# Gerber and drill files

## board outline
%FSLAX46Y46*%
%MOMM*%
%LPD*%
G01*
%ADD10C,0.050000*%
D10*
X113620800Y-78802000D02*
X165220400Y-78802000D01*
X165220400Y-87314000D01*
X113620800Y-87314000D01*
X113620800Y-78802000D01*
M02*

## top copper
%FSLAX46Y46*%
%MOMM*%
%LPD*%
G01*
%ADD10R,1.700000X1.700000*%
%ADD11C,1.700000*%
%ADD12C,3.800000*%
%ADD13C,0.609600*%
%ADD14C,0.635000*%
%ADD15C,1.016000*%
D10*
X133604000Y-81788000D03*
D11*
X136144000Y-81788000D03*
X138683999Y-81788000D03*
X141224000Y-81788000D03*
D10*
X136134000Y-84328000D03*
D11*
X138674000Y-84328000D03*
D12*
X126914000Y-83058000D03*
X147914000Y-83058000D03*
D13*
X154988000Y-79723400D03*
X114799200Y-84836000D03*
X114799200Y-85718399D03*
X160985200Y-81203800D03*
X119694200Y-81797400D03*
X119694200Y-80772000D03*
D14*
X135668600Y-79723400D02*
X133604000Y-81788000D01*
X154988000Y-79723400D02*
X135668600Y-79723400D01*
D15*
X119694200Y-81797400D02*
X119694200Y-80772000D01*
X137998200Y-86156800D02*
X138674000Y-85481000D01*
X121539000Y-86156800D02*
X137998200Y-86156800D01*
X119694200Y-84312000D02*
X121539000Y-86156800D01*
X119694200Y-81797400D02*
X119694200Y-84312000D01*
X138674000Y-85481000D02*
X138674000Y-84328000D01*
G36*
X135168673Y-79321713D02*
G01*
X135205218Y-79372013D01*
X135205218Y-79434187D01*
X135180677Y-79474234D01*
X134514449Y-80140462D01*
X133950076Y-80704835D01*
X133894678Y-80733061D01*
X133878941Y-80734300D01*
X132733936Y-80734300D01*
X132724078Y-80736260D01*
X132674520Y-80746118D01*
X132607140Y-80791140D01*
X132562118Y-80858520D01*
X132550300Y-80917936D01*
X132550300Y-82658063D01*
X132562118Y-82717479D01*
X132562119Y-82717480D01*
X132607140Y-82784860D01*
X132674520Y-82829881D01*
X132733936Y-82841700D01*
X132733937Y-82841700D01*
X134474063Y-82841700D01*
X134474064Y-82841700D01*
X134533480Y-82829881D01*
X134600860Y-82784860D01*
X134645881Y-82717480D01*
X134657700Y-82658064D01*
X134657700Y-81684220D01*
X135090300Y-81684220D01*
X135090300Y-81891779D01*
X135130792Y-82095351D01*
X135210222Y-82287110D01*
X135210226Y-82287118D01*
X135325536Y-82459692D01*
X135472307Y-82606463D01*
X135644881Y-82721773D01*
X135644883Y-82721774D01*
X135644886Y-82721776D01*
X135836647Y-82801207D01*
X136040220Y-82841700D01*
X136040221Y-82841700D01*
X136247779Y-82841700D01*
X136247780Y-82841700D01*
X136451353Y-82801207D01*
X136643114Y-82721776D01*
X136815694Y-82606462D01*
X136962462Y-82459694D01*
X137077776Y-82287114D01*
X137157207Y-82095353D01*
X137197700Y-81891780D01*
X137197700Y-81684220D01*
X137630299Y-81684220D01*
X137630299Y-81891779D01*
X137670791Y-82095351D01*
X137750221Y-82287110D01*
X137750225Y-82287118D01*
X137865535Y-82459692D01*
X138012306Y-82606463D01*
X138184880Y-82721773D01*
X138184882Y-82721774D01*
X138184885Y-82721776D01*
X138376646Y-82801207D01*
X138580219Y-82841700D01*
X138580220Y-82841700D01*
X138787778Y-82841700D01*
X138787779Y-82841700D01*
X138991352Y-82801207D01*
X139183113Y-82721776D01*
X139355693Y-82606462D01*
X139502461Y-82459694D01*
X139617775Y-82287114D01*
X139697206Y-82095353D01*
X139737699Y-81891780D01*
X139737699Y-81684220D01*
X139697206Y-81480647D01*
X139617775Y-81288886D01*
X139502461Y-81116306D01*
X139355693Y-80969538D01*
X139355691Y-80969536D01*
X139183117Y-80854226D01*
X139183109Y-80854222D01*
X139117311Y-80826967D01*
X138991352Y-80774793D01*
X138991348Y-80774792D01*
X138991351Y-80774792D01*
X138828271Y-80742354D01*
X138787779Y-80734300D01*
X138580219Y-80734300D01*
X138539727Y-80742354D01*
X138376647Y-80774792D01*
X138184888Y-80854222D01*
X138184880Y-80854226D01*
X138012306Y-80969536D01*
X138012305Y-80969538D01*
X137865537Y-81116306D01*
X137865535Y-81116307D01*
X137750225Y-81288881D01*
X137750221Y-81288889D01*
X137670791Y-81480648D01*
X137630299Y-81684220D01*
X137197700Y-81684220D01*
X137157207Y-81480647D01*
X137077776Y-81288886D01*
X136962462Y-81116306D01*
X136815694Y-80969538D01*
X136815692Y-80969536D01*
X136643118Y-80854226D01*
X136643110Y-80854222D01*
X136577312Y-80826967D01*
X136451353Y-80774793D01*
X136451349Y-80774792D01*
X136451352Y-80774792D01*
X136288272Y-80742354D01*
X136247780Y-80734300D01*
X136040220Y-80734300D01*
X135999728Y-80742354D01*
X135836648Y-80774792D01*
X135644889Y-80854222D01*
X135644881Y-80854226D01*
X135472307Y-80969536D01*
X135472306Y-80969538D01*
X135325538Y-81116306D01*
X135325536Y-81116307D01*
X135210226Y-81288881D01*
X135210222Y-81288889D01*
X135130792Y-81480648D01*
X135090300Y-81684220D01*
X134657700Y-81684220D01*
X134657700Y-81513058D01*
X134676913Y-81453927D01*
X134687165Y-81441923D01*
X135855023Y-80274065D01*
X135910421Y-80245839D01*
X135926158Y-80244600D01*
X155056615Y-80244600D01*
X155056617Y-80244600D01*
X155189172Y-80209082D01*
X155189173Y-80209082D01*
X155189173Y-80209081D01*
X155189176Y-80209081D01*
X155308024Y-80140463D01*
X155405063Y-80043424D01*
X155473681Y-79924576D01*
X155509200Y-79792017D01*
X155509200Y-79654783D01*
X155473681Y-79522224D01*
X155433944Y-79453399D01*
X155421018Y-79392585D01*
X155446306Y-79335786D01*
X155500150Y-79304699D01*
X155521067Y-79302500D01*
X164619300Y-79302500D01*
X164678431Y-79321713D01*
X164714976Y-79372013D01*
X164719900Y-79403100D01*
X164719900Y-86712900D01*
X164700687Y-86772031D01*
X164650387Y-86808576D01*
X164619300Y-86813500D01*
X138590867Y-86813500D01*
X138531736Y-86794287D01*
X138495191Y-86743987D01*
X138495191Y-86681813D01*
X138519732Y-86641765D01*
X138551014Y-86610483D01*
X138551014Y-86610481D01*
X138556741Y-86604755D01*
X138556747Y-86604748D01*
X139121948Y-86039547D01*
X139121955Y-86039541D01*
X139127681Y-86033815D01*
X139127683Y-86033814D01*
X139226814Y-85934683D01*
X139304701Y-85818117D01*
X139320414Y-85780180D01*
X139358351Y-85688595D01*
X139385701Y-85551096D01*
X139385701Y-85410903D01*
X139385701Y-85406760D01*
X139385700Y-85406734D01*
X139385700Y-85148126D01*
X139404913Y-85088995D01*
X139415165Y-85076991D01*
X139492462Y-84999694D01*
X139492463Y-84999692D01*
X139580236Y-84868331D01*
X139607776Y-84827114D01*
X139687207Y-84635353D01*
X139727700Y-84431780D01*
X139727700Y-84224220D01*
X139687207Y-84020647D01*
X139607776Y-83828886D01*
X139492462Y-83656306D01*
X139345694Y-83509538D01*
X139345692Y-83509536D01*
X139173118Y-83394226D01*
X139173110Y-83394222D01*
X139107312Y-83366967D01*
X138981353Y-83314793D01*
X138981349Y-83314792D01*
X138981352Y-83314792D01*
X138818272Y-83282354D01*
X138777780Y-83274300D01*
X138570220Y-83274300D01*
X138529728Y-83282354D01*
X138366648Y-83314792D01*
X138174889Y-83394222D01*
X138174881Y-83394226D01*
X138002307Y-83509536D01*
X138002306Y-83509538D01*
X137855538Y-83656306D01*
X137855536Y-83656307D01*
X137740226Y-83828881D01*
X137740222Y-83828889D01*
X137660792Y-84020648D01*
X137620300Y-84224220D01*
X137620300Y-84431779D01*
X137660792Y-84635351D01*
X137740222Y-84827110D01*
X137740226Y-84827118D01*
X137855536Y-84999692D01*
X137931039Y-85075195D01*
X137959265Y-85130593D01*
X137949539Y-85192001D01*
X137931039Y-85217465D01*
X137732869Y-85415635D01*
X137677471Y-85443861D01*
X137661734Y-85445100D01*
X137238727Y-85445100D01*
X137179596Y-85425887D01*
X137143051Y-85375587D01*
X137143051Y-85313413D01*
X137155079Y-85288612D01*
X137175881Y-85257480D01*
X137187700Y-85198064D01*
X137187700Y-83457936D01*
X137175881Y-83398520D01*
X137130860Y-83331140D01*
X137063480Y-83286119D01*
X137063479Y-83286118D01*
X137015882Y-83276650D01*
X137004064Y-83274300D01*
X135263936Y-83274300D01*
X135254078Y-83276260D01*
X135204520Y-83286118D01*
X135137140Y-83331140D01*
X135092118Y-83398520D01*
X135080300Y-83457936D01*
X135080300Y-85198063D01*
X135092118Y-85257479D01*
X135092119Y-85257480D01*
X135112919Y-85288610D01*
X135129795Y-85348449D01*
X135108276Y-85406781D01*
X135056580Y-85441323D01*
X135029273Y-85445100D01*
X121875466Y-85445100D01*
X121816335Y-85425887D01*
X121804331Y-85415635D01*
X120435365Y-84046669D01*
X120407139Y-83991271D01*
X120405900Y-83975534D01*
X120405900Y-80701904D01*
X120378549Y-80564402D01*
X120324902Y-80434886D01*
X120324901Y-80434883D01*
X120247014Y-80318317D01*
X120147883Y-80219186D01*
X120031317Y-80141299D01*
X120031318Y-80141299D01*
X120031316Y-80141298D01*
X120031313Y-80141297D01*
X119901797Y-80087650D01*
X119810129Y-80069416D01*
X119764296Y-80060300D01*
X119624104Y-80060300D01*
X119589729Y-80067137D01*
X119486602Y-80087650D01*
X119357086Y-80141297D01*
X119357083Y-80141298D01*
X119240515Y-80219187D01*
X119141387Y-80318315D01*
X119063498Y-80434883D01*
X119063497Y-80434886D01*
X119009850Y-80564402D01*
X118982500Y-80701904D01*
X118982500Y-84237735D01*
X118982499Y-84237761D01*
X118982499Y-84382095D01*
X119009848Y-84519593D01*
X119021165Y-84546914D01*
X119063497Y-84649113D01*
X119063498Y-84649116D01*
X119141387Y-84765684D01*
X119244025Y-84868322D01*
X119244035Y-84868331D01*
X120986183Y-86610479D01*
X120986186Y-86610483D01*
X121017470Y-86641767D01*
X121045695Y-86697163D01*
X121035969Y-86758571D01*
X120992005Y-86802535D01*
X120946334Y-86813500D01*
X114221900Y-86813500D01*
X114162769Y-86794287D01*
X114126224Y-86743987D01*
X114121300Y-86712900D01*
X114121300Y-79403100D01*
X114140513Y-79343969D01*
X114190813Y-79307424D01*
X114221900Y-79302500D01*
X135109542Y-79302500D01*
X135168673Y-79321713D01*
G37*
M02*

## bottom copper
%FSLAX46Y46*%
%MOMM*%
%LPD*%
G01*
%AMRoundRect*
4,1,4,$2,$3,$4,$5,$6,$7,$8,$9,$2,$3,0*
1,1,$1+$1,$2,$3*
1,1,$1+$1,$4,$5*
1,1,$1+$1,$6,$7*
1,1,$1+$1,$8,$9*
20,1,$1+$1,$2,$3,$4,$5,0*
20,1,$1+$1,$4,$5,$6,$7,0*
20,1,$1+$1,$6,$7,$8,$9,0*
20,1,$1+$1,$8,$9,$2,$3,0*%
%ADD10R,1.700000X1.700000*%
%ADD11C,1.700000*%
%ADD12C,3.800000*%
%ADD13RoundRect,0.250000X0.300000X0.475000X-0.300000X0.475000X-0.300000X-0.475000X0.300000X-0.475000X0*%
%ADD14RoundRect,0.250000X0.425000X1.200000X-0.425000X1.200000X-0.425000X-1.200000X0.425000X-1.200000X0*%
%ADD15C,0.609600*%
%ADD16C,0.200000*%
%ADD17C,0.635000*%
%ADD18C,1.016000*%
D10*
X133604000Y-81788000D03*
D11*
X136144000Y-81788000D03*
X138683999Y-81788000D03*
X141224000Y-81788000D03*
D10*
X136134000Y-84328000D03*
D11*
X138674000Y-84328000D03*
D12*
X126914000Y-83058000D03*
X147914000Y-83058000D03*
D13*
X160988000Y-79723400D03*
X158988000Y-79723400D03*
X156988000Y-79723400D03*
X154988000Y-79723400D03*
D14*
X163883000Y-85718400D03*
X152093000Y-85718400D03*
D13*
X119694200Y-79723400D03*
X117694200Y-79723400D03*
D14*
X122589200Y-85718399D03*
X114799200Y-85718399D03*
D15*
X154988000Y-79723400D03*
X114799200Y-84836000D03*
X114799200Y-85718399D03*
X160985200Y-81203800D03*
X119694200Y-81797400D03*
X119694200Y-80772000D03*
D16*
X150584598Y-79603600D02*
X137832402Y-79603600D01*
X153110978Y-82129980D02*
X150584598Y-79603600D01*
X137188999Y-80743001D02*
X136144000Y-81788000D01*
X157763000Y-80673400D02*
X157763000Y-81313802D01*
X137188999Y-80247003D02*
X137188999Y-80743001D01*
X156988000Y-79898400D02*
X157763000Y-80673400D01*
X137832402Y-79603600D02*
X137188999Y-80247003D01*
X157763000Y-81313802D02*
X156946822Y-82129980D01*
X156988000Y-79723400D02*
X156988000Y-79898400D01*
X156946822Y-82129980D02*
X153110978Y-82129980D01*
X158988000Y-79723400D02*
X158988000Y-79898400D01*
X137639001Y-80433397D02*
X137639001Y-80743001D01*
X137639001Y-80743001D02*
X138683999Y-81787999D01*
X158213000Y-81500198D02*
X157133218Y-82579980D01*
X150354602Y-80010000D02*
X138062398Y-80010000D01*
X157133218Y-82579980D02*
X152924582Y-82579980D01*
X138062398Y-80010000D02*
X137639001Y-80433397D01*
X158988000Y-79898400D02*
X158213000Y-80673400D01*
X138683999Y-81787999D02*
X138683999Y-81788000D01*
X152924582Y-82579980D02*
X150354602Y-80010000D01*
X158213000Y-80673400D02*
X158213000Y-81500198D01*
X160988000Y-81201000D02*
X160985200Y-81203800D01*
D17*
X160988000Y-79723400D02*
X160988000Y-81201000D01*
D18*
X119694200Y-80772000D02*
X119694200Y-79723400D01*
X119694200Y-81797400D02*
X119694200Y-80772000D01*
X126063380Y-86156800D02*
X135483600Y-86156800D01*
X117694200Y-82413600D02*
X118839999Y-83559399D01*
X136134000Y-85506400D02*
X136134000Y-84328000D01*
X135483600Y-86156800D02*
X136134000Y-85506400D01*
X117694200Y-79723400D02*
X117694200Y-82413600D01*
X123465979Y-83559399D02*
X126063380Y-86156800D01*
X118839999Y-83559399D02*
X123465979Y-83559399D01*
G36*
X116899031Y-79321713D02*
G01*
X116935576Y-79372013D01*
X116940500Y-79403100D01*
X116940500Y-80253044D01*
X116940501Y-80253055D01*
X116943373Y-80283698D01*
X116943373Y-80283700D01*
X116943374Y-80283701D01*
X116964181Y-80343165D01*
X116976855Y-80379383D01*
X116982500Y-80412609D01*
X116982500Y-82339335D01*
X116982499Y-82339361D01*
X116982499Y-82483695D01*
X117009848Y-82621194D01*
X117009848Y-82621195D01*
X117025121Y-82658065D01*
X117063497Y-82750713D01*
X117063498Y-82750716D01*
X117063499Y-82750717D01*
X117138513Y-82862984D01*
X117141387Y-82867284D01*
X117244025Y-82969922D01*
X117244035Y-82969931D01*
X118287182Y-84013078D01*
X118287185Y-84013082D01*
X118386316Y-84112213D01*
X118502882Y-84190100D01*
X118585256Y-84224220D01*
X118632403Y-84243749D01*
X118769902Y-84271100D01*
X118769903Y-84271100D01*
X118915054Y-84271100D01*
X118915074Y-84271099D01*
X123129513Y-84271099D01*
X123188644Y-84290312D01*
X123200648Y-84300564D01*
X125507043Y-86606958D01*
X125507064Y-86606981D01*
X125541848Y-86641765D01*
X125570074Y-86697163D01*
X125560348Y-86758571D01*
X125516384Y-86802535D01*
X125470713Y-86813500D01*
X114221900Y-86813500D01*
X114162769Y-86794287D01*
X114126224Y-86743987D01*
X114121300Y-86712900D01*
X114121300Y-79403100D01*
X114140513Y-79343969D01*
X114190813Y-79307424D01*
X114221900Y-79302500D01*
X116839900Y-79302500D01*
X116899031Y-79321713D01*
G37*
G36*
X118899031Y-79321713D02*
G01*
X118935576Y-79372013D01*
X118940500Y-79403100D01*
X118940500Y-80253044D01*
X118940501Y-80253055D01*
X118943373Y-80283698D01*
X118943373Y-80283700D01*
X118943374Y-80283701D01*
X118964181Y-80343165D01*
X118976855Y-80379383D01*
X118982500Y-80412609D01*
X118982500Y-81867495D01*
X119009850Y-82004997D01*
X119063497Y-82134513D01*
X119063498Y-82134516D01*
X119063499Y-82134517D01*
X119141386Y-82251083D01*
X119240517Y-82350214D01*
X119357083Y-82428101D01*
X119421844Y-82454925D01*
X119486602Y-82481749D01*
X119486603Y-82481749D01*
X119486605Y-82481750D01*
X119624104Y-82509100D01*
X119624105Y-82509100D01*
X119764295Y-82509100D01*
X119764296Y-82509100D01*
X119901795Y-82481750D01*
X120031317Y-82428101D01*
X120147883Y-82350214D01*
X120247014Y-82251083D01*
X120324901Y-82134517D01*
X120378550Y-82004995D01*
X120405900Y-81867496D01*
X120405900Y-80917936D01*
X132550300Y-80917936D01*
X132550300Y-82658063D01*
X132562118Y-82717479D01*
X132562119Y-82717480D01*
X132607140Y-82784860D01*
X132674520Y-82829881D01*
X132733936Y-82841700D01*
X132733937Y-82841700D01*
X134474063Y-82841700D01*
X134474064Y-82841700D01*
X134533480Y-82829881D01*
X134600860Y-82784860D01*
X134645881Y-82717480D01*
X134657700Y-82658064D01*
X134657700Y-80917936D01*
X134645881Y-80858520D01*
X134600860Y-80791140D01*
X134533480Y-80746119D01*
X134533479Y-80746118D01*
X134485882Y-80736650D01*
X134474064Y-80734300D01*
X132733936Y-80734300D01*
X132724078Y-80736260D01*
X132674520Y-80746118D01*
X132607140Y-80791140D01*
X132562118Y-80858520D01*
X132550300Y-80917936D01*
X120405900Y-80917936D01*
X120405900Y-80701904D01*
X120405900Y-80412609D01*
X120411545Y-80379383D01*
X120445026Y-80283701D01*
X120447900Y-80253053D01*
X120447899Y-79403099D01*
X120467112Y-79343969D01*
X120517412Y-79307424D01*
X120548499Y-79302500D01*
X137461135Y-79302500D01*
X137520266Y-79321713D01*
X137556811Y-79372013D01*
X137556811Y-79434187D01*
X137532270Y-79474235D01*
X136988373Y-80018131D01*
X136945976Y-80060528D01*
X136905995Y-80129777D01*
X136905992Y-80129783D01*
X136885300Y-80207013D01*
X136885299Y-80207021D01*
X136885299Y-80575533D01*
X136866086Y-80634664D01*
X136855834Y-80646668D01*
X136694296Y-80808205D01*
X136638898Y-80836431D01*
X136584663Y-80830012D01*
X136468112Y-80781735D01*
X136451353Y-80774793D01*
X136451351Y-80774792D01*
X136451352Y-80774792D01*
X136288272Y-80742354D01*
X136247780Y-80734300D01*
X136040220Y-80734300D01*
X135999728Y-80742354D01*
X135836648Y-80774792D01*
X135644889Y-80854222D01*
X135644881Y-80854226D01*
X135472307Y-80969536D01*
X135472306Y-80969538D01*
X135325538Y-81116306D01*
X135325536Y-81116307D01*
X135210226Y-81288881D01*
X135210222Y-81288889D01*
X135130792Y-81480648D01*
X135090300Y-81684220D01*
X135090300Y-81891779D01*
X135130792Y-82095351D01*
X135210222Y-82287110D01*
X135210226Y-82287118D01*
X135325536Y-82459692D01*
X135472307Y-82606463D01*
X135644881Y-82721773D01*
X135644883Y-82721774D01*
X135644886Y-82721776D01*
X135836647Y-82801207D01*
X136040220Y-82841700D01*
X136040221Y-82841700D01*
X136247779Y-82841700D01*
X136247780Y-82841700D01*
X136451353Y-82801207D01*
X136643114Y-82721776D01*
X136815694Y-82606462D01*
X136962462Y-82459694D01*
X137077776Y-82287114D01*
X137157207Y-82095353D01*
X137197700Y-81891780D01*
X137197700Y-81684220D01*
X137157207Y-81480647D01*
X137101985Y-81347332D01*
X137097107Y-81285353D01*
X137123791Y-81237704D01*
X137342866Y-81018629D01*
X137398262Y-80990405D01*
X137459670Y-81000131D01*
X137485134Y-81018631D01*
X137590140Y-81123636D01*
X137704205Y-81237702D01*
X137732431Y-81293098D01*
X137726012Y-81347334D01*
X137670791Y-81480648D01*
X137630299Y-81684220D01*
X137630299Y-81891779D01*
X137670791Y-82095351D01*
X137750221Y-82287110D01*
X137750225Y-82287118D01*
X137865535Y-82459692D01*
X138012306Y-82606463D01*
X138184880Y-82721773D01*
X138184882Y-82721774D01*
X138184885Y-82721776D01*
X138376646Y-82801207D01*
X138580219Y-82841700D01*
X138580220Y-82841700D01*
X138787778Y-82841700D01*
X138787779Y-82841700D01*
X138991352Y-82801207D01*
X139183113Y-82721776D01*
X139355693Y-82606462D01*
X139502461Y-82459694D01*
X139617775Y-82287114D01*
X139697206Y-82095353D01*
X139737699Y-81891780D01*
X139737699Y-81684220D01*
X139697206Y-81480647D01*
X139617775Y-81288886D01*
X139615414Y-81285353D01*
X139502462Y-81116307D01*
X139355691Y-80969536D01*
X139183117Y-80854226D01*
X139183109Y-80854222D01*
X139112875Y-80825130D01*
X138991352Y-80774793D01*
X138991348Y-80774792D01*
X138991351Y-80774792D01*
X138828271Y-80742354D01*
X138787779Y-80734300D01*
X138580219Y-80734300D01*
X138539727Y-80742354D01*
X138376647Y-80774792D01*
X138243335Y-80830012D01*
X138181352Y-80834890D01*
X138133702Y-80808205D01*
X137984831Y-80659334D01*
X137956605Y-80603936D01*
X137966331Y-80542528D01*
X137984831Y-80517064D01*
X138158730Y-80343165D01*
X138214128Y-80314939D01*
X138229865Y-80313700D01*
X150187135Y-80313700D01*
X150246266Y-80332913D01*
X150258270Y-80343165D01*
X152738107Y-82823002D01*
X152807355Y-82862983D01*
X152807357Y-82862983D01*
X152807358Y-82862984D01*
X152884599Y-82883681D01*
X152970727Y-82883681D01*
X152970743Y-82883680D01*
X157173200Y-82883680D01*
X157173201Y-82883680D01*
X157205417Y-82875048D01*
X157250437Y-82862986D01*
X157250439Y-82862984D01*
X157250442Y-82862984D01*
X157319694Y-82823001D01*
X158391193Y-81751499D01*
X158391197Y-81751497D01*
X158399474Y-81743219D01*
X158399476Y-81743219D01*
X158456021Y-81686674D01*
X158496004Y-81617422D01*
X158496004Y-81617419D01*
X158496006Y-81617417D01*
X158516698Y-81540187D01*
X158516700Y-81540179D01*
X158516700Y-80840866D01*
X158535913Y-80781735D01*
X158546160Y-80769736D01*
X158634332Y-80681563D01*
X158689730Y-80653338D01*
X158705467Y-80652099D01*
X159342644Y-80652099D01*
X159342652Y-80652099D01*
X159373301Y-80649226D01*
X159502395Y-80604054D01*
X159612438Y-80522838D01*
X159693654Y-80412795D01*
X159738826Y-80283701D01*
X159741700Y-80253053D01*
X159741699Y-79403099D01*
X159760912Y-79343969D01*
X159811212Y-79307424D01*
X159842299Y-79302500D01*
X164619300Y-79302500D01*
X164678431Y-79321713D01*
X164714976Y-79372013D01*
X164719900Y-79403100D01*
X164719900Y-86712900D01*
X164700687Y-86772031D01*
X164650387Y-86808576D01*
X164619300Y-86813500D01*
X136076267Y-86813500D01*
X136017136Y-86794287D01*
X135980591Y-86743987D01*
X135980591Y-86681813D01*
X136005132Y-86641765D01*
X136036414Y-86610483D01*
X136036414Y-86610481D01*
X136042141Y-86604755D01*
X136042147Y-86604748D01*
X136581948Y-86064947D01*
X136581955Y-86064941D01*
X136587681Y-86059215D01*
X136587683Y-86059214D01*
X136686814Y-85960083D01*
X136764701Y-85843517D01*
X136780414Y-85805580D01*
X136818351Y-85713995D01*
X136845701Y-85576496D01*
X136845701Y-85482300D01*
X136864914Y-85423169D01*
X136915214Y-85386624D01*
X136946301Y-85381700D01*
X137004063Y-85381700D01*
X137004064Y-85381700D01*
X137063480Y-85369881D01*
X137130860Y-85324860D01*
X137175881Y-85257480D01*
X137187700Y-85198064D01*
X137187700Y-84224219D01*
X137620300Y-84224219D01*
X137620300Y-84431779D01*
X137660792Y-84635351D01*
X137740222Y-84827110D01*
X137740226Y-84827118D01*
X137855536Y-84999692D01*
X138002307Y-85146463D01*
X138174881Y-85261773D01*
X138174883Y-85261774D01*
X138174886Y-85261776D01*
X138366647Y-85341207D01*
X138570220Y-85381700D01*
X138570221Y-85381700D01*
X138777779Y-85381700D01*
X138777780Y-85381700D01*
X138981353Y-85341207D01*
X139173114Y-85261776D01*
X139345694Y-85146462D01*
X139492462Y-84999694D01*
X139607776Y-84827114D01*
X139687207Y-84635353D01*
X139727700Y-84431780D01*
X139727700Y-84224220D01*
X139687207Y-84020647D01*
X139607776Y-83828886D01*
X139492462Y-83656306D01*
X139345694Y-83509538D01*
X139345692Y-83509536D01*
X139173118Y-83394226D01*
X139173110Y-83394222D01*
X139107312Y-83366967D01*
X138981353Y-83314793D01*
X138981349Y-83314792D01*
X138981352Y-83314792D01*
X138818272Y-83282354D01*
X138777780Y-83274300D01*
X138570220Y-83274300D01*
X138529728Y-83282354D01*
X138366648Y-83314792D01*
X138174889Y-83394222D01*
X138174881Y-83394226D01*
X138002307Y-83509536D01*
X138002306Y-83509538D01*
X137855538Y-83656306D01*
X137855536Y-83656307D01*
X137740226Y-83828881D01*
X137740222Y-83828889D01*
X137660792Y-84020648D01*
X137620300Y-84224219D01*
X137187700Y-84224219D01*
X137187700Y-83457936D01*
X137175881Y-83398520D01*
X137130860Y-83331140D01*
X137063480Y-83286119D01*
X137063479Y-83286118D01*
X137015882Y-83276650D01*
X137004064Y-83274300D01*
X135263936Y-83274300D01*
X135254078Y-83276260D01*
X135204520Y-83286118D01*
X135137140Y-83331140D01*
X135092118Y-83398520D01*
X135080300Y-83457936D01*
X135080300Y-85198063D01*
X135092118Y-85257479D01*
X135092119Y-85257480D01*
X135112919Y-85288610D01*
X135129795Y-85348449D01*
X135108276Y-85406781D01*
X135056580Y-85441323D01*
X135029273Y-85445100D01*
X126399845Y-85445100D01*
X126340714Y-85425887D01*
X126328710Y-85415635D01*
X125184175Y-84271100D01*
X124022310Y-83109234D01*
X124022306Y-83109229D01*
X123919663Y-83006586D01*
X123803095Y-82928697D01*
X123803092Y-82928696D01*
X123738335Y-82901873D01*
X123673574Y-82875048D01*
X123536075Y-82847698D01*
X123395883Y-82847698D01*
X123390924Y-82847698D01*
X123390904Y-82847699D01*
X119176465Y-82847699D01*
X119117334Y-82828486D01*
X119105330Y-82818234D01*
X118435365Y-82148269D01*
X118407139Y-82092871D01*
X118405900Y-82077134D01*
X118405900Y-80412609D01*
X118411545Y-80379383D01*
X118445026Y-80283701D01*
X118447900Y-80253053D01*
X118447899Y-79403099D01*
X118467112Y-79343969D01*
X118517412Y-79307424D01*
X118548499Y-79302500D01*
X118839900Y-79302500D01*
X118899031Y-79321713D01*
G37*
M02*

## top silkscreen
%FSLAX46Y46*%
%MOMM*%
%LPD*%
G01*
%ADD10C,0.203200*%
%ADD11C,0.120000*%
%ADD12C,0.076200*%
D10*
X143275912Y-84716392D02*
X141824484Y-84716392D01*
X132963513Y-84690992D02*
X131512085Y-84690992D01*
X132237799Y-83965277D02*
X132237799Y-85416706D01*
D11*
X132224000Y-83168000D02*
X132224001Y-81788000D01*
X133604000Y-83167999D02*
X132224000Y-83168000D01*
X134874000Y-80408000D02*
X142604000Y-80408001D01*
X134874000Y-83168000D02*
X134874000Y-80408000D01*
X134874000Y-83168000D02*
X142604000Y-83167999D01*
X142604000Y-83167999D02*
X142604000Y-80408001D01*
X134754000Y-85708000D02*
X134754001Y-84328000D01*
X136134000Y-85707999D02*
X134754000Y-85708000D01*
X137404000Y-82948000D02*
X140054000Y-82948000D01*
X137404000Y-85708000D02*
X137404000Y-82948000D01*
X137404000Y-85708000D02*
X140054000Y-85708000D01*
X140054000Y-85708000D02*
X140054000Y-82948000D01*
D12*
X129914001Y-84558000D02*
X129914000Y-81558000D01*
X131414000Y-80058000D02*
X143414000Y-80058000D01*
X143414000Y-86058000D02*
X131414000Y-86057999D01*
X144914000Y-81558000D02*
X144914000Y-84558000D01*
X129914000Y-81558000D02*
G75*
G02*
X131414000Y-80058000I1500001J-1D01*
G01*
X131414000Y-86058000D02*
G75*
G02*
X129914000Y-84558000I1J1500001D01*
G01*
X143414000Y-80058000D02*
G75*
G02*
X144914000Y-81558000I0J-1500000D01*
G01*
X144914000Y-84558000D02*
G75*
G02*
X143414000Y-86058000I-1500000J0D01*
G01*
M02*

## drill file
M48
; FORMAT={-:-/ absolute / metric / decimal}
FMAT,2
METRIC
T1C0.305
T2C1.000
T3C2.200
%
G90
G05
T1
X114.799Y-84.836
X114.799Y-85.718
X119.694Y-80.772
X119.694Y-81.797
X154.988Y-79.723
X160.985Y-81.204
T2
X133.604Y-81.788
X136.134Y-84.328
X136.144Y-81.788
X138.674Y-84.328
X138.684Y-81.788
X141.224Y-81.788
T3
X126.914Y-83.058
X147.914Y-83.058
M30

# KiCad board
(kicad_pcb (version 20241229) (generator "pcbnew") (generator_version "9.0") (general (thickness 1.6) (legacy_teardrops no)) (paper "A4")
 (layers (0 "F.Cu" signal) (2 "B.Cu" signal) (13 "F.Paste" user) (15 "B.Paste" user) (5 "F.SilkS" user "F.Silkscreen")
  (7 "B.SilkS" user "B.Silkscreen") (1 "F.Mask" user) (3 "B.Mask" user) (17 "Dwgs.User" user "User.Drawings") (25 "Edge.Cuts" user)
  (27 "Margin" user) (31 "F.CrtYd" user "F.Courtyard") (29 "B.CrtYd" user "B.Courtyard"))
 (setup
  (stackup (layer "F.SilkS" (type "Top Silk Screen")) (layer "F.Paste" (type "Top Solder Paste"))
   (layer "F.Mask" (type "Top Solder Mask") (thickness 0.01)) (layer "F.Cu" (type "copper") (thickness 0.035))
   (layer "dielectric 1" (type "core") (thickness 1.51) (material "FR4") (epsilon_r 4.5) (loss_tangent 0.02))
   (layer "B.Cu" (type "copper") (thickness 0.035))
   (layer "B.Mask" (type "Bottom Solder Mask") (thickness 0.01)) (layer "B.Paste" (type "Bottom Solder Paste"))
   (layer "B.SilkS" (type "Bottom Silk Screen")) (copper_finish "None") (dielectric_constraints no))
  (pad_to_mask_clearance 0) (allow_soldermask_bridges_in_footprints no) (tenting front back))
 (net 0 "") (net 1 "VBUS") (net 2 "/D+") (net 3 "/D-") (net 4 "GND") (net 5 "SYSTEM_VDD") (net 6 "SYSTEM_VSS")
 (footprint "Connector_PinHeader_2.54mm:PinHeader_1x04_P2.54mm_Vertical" (layer "F.Cu") (at 133.604 81.788 90)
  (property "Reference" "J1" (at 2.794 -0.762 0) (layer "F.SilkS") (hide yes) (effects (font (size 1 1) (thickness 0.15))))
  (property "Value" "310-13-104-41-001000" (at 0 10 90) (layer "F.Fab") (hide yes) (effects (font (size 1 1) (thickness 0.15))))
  (fp_line (start -1.38 -1.38) (end 0 -1.379999) (stroke (width 0.12) (type solid)) (layer "F.SilkS"))
  (fp_line (start -1.379999 0) (end -1.38 -1.38) (stroke (width 0.12) (type solid)) (layer "F.SilkS"))
  (fp_line (start 1.38 1.27) (end 1.379999 9) (stroke (width 0.12) (type solid)) (layer "F.SilkS"))
  (fp_line (start -1.38 1.27) (end 1.38 1.27) (stroke (width 0.12) (type solid)) (layer "F.SilkS"))
  (fp_line (start -1.38 1.27) (end -1.379999 9) (stroke (width 0.12) (type solid)) (layer "F.SilkS"))
  (fp_line (start -1.379999 9) (end 1.379999 9) (stroke (width 0.12) (type solid)) (layer "F.SilkS"))
  (pad "1" thru_hole rect (at 0 0 90) (size 1.7 1.7) (drill 1) (layers "*.Cu" "*.Mask") (remove_unused_layers no) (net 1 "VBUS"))
  (pad "2" thru_hole circle (at 0 2.54 90) (size 1.7 1.7) (drill 1) (layers "*.Cu" "*.Mask") (remove_unused_layers no) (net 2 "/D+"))
  (pad "3" thru_hole circle (at 0 5.079999 90) (size 1.7 1.7) (drill 1) (layers "*.Cu" "*.Mask") (remove_unused_layers no) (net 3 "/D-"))
  (pad "4" thru_hole circle (at 0 7.62 90) (size 1.7 1.7) (drill 1) (layers "*.Cu" "*.Mask") (remove_unused_layers no) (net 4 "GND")))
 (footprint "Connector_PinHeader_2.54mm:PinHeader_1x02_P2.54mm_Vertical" (layer "F.Cu") (at 136.134 84.328 90)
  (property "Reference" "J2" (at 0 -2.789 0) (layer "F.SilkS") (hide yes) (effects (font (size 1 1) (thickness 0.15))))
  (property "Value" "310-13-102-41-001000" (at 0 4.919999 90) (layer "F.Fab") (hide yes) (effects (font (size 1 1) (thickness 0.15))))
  (fp_line (start -1.38 -1.38) (end 0 -1.379999) (stroke (width 0.12) (type solid)) (layer "F.SilkS"))
  (fp_line (start -1.379999 0) (end -1.38 -1.38) (stroke (width 0.12) (type solid)) (layer "F.SilkS"))
  (fp_line (start 1.38 1.27) (end 1.38 3.92) (stroke (width 0.12) (type solid)) (layer "F.SilkS"))
  (fp_line (start -1.38 1.27) (end 1.38 1.27) (stroke (width 0.12) (type solid)) (layer "F.SilkS"))
  (fp_line (start -1.38 1.27) (end -1.38 3.92) (stroke (width 0.12) (type solid)) (layer "F.SilkS"))
  (fp_line (start -1.38 3.92) (end 1.38 3.92) (stroke (width 0.12) (type solid)) (layer "F.SilkS"))
  (pad "1" thru_hole rect (at 0 0 90) (size 1.7 1.7) (drill 1) (layers "*.Cu" "*.Mask") (remove_unused_layers no) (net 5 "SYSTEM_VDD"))
  (pad "2" thru_hole circle (at 0 2.54 90) (size 1.7 1.7) (drill 1) (layers "*.Cu" "*.Mask") (remove_unused_layers no) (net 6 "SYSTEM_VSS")))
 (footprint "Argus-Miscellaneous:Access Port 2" (layer "F.Cu") (at 137.414 83.058)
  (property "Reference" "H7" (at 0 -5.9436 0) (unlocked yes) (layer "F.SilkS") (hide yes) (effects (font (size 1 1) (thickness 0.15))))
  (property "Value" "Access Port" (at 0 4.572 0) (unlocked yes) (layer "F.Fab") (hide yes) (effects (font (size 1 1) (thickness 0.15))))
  (fp_line (start -7.499999 1.5) (end -7.5 -1.5) (stroke (width 0.0762) (type solid)) (layer "F.SilkS"))
  (fp_line (start -6 -3) (end 6 -3) (stroke (width 0.0762) (type solid)) (layer "F.SilkS"))
  (fp_line (start 6 3) (end -6 2.999999) (stroke (width 0.0762) (type solid)) (layer "F.SilkS"))
  (fp_line (start 7.5 -1.5) (end 7.5 1.5) (stroke (width 0.0762) (type solid)) (layer "F.SilkS"))
  (fp_arc (start -7.5 -1.5) (mid -7.06066 -2.56066) (end -6 -3) (stroke (width 0.0762) (type solid)) (layer "F.SilkS"))
  (fp_arc (start -6 3) (mid -7.06066 2.56066) (end -7.5 1.5) (stroke (width 0.0762) (type solid)) (layer "F.SilkS"))
  (fp_arc (start 6 -3) (mid 7.06066 -2.56066) (end 7.5 -1.5) (stroke (width 0.0762) (type solid)) (layer "F.SilkS"))
  (fp_arc (start 7.5 1.5) (mid 7.06066 2.56066) (end 6 3) (stroke (width 0.0762) (type solid)) (layer "F.SilkS"))
  (pad "1" thru_hole circle (at -10.5 0) (size 3.8 3.8) (drill 2.2) (layers "*.Cu" "*.Mask") (remove_unused_layers no) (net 4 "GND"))
  (pad "1" thru_hole circle (at 10.5 0) (size 3.8 3.8) (drill 2.2) (layers "*.Cu" "*.Mask") (remove_unused_layers no) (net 4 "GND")))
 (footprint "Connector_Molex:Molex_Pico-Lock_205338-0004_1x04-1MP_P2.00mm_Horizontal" (layer "B.Cu") (at 157.988 83.0834 180)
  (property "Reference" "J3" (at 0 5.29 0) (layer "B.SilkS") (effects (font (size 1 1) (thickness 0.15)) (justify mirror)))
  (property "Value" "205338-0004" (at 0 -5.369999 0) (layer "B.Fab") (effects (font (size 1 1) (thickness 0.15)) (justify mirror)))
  (pad "1" smd roundrect (at -3 3.36 180) (size 1.1 1.45) (layers "B.Cu" "B.Mask" "B.Paste") (roundrect_rratio 0.227273) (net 4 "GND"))
  (pad "2" smd roundrect (at -1 3.36 180) (size 1.1 1.45) (layers "B.Cu" "B.Mask" "B.Paste") (roundrect_rratio 0.227273) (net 3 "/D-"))
  (pad "3" smd roundrect (at 1 3.36 180) (size 1.1 1.45) (layers "B.Cu" "B.Mask" "B.Paste") (roundrect_rratio 0.227273) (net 2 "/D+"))
  (pad "4" smd roundrect (at 3 3.36 180) (size 1.1 1.45) (layers "B.Cu" "B.Mask" "B.Paste") (roundrect_rratio 0.227273) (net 1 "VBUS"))
  (pad "MP" smd roundrect (at -5.895 -2.635 180) (size 1.35 2.9) (layers "B.Cu" "B.Mask" "B.Paste") (roundrect_rratio 0.185185)
   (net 4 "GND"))
  (pad "MP" smd roundrect (at 5.895 -2.635 180) (size 1.35 2.9) (layers "B.Cu" "B.Mask" "B.Paste") (roundrect_rratio 0.185185) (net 4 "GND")))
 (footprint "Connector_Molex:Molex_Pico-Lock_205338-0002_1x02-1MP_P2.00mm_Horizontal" (layer "B.Cu") (at 118.6942 83.0834 180)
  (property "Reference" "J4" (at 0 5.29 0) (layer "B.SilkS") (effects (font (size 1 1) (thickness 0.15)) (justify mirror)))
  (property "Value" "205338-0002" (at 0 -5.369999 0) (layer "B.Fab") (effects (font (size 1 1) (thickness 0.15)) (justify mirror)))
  (pad "1" smd roundrect (at -1 3.36 180) (size 1.1 1.45) (layers "B.Cu" "B.Mask" "B.Paste") (roundrect_rratio 0.227273)
   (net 6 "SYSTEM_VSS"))
  (pad "2" smd roundrect (at 1 3.36 180) (size 1.1 1.45) (layers "B.Cu" "B.Mask" "B.Paste") (roundrect_rratio 0.227273) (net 5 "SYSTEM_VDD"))
  (pad "MP" smd roundrect (at -3.895 -2.634999 180) (size 1.35 2.9) (layers "B.Cu" "B.Mask" "B.Paste") (roundrect_rratio 0.185185)
   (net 4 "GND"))
  (pad "MP" smd roundrect (at 3.895 -2.634999 180) (size 1.35 2.9) (layers "B.Cu" "B.Mask" "B.Paste") (roundrect_rratio 0.185185)
   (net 4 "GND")))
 (gr_rect (start 113.6208 78.802) (end 165.2204 87.314) (stroke (width 0.05) (type solid)) (fill no) (layer "Edge.Cuts"))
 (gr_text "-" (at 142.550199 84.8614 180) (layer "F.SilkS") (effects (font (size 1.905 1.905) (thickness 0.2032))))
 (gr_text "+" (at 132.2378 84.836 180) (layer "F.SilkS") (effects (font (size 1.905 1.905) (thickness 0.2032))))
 (segment (start 150.584598 79.6036) (end 137.832402 79.6036) (width 0.2) (layer "B.Cu") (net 2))
 (segment (start 153.110978 82.12998) (end 150.584598 79.6036) (width 0.2) (layer "B.Cu") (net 2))
 (segment (start 137.188999 80.743001) (end 136.144 81.788) (width 0.2) (layer "B.Cu") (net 2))
 (segment (start 157.763 80.6734) (end 157.763 81.313802) (width 0.2) (layer "B.Cu") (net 2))
 (segment (start 137.188999 80.247003) (end 137.188999 80.743001) (width 0.2) (layer "B.Cu") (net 2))
 (segment (start 156.988 79.8984) (end 157.763 80.6734) (width 0.2) (layer "B.Cu") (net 2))
 (segment (start 137.832402 79.6036) (end 137.188999 80.247003) (width 0.2) (layer "B.Cu") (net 2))
 (segment (start 157.763 81.313802) (end 156.946822 82.12998) (width 0.2) (layer "B.Cu") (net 2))
 (segment (start 156.988 79.7234) (end 156.988 79.8984) (width 0.2) (layer "B.Cu") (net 2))
 (segment (start 156.946822 82.12998) (end 153.110978 82.12998) (width 0.2) (layer "B.Cu") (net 2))
 (segment (start 135.6686 79.7234) (end 133.604 81.788) (width 0.635) (layer "F.Cu") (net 1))
 (segment (start 154.988 79.7234) (end 135.6686 79.7234) (width 0.635) (layer "F.Cu") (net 1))
 (via (at 154.988 79.7234) (size 0.6096) (drill 0.3048) (layers "F.Cu" "B.Cu") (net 1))
 (segment (start 158.988 79.7234) (end 158.988 79.8984) (width 0.2) (layer "B.Cu") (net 3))
 (segment (start 137.639001 80.433397) (end 137.639001 80.743001) (width 0.2) (layer "B.Cu") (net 3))
 (segment (start 137.639001 80.743001) (end 138.683999 81.787999) (width 0.2) (layer "B.Cu") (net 3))
 (segment (start 158.213 81.500198) (end 157.133218 82.57998) (width 0.2) (layer "B.Cu") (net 3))
 (segment (start 150.354602 80.01) (end 138.062398 80.01) (width 0.2) (layer "B.Cu") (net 3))
 (segment (start 157.133218 82.57998) (end 152.924582 82.57998) (width 0.2) (layer "B.Cu") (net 3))
 (segment (start 138.062398 80.01) (end 137.639001 80.433397) (width 0.2) (layer "B.Cu") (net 3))
 (segment (start 158.988 79.8984) (end 158.213 80.6734) (width 0.2) (layer "B.Cu") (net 3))
 (segment (start 138.683999 81.787999) (end 138.683999 81.788) (width 0.2) (layer "B.Cu") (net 3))
 (segment (start 152.924582 82.57998) (end 150.354602 80.01) (width 0.2) (layer "B.Cu") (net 3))
 (segment (start 158.213 80.6734) (end 158.213 81.500198) (width 0.2) (layer "B.Cu") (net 3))
 (via (at 114.7992 84.836) (size 0.6096) (drill 0.3048) (layers "F.Cu" "B.Cu") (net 4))
 (via (at 114.7992 85.718399) (size 0.6096) (drill 0.3048) (layers "F.Cu" "B.Cu") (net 4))
 (via (at 160.9852 81.2038) (size 0.6096) (drill 0.3048) (layers "F.Cu" "B.Cu") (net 4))
 (segment (start 160.988 81.201) (end 160.9852 81.2038) (width 0.2) (layer "B.Cu") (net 4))
 (segment (start 160.988 79.7234) (end 160.988 81.201) (width 0.635) (layer "B.Cu") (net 4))
 (segment (start 119.6942 81.7974) (end 119.6942 80.772) (width 1.016) (layer "F.Cu") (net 6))
 (segment (start 137.9982 86.1568) (end 138.674 85.481) (width 1.016) (layer "F.Cu") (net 6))
 (segment (start 121.539 86.1568) (end 137.9982 86.1568) (width 1.016) (layer "F.Cu") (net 6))
 (segment (start 119.6942 84.312) (end 121.539 86.1568) (width 1.016) (layer "F.Cu") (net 6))
 (segment (start 119.6942 81.7974) (end 119.6942 84.312) (width 1.016) (layer "F.Cu") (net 6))
 (segment (start 138.674 85.481) (end 138.674 84.328) (width 1.016) (layer "F.Cu") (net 6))
 (via (at 119.6942 81.7974) (size 0.6096) (drill 0.3048) (layers "F.Cu" "B.Cu") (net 6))
 (via (at 119.6942 80.772) (size 0.6096) (drill 0.3048) (layers "F.Cu" "B.Cu") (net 6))
 (segment (start 119.6942 80.772) (end 119.6942 79.7234) (width 1.016) (layer "B.Cu") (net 6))
 (segment (start 119.6942 81.7974) (end 119.6942 80.772) (width 1.016) (layer "B.Cu") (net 6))
 (segment (start 126.06338 86.1568) (end 135.4836 86.1568) (width 1.016) (layer "B.Cu") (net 5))
 (segment (start 117.6942 82.4136) (end 118.839999 83.559399) (width 1.016) (layer "B.Cu") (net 5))
 (segment (start 136.134 85.5064) (end 136.134 84.328) (width 1.016) (layer "B.Cu") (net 5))
 (segment (start 135.4836 86.1568) (end 136.134 85.5064) (width 1.016) (layer "B.Cu") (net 5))
 (segment (start 117.6942 79.7234) (end 117.6942 82.4136) (width 1.016) (layer "B.Cu") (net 5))
 (segment (start 123.465979 83.559399) (end 126.06338 86.1568) (width 1.016) (layer "B.Cu") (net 5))
 (segment (start 118.839999 83.559399) (end 123.465979 83.559399) (width 1.016) (layer "B.Cu") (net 5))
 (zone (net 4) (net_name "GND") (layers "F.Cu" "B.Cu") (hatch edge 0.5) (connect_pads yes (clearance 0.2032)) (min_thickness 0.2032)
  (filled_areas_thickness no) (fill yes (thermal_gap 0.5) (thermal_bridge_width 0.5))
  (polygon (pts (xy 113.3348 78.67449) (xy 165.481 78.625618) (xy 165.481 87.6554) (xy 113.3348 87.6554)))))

